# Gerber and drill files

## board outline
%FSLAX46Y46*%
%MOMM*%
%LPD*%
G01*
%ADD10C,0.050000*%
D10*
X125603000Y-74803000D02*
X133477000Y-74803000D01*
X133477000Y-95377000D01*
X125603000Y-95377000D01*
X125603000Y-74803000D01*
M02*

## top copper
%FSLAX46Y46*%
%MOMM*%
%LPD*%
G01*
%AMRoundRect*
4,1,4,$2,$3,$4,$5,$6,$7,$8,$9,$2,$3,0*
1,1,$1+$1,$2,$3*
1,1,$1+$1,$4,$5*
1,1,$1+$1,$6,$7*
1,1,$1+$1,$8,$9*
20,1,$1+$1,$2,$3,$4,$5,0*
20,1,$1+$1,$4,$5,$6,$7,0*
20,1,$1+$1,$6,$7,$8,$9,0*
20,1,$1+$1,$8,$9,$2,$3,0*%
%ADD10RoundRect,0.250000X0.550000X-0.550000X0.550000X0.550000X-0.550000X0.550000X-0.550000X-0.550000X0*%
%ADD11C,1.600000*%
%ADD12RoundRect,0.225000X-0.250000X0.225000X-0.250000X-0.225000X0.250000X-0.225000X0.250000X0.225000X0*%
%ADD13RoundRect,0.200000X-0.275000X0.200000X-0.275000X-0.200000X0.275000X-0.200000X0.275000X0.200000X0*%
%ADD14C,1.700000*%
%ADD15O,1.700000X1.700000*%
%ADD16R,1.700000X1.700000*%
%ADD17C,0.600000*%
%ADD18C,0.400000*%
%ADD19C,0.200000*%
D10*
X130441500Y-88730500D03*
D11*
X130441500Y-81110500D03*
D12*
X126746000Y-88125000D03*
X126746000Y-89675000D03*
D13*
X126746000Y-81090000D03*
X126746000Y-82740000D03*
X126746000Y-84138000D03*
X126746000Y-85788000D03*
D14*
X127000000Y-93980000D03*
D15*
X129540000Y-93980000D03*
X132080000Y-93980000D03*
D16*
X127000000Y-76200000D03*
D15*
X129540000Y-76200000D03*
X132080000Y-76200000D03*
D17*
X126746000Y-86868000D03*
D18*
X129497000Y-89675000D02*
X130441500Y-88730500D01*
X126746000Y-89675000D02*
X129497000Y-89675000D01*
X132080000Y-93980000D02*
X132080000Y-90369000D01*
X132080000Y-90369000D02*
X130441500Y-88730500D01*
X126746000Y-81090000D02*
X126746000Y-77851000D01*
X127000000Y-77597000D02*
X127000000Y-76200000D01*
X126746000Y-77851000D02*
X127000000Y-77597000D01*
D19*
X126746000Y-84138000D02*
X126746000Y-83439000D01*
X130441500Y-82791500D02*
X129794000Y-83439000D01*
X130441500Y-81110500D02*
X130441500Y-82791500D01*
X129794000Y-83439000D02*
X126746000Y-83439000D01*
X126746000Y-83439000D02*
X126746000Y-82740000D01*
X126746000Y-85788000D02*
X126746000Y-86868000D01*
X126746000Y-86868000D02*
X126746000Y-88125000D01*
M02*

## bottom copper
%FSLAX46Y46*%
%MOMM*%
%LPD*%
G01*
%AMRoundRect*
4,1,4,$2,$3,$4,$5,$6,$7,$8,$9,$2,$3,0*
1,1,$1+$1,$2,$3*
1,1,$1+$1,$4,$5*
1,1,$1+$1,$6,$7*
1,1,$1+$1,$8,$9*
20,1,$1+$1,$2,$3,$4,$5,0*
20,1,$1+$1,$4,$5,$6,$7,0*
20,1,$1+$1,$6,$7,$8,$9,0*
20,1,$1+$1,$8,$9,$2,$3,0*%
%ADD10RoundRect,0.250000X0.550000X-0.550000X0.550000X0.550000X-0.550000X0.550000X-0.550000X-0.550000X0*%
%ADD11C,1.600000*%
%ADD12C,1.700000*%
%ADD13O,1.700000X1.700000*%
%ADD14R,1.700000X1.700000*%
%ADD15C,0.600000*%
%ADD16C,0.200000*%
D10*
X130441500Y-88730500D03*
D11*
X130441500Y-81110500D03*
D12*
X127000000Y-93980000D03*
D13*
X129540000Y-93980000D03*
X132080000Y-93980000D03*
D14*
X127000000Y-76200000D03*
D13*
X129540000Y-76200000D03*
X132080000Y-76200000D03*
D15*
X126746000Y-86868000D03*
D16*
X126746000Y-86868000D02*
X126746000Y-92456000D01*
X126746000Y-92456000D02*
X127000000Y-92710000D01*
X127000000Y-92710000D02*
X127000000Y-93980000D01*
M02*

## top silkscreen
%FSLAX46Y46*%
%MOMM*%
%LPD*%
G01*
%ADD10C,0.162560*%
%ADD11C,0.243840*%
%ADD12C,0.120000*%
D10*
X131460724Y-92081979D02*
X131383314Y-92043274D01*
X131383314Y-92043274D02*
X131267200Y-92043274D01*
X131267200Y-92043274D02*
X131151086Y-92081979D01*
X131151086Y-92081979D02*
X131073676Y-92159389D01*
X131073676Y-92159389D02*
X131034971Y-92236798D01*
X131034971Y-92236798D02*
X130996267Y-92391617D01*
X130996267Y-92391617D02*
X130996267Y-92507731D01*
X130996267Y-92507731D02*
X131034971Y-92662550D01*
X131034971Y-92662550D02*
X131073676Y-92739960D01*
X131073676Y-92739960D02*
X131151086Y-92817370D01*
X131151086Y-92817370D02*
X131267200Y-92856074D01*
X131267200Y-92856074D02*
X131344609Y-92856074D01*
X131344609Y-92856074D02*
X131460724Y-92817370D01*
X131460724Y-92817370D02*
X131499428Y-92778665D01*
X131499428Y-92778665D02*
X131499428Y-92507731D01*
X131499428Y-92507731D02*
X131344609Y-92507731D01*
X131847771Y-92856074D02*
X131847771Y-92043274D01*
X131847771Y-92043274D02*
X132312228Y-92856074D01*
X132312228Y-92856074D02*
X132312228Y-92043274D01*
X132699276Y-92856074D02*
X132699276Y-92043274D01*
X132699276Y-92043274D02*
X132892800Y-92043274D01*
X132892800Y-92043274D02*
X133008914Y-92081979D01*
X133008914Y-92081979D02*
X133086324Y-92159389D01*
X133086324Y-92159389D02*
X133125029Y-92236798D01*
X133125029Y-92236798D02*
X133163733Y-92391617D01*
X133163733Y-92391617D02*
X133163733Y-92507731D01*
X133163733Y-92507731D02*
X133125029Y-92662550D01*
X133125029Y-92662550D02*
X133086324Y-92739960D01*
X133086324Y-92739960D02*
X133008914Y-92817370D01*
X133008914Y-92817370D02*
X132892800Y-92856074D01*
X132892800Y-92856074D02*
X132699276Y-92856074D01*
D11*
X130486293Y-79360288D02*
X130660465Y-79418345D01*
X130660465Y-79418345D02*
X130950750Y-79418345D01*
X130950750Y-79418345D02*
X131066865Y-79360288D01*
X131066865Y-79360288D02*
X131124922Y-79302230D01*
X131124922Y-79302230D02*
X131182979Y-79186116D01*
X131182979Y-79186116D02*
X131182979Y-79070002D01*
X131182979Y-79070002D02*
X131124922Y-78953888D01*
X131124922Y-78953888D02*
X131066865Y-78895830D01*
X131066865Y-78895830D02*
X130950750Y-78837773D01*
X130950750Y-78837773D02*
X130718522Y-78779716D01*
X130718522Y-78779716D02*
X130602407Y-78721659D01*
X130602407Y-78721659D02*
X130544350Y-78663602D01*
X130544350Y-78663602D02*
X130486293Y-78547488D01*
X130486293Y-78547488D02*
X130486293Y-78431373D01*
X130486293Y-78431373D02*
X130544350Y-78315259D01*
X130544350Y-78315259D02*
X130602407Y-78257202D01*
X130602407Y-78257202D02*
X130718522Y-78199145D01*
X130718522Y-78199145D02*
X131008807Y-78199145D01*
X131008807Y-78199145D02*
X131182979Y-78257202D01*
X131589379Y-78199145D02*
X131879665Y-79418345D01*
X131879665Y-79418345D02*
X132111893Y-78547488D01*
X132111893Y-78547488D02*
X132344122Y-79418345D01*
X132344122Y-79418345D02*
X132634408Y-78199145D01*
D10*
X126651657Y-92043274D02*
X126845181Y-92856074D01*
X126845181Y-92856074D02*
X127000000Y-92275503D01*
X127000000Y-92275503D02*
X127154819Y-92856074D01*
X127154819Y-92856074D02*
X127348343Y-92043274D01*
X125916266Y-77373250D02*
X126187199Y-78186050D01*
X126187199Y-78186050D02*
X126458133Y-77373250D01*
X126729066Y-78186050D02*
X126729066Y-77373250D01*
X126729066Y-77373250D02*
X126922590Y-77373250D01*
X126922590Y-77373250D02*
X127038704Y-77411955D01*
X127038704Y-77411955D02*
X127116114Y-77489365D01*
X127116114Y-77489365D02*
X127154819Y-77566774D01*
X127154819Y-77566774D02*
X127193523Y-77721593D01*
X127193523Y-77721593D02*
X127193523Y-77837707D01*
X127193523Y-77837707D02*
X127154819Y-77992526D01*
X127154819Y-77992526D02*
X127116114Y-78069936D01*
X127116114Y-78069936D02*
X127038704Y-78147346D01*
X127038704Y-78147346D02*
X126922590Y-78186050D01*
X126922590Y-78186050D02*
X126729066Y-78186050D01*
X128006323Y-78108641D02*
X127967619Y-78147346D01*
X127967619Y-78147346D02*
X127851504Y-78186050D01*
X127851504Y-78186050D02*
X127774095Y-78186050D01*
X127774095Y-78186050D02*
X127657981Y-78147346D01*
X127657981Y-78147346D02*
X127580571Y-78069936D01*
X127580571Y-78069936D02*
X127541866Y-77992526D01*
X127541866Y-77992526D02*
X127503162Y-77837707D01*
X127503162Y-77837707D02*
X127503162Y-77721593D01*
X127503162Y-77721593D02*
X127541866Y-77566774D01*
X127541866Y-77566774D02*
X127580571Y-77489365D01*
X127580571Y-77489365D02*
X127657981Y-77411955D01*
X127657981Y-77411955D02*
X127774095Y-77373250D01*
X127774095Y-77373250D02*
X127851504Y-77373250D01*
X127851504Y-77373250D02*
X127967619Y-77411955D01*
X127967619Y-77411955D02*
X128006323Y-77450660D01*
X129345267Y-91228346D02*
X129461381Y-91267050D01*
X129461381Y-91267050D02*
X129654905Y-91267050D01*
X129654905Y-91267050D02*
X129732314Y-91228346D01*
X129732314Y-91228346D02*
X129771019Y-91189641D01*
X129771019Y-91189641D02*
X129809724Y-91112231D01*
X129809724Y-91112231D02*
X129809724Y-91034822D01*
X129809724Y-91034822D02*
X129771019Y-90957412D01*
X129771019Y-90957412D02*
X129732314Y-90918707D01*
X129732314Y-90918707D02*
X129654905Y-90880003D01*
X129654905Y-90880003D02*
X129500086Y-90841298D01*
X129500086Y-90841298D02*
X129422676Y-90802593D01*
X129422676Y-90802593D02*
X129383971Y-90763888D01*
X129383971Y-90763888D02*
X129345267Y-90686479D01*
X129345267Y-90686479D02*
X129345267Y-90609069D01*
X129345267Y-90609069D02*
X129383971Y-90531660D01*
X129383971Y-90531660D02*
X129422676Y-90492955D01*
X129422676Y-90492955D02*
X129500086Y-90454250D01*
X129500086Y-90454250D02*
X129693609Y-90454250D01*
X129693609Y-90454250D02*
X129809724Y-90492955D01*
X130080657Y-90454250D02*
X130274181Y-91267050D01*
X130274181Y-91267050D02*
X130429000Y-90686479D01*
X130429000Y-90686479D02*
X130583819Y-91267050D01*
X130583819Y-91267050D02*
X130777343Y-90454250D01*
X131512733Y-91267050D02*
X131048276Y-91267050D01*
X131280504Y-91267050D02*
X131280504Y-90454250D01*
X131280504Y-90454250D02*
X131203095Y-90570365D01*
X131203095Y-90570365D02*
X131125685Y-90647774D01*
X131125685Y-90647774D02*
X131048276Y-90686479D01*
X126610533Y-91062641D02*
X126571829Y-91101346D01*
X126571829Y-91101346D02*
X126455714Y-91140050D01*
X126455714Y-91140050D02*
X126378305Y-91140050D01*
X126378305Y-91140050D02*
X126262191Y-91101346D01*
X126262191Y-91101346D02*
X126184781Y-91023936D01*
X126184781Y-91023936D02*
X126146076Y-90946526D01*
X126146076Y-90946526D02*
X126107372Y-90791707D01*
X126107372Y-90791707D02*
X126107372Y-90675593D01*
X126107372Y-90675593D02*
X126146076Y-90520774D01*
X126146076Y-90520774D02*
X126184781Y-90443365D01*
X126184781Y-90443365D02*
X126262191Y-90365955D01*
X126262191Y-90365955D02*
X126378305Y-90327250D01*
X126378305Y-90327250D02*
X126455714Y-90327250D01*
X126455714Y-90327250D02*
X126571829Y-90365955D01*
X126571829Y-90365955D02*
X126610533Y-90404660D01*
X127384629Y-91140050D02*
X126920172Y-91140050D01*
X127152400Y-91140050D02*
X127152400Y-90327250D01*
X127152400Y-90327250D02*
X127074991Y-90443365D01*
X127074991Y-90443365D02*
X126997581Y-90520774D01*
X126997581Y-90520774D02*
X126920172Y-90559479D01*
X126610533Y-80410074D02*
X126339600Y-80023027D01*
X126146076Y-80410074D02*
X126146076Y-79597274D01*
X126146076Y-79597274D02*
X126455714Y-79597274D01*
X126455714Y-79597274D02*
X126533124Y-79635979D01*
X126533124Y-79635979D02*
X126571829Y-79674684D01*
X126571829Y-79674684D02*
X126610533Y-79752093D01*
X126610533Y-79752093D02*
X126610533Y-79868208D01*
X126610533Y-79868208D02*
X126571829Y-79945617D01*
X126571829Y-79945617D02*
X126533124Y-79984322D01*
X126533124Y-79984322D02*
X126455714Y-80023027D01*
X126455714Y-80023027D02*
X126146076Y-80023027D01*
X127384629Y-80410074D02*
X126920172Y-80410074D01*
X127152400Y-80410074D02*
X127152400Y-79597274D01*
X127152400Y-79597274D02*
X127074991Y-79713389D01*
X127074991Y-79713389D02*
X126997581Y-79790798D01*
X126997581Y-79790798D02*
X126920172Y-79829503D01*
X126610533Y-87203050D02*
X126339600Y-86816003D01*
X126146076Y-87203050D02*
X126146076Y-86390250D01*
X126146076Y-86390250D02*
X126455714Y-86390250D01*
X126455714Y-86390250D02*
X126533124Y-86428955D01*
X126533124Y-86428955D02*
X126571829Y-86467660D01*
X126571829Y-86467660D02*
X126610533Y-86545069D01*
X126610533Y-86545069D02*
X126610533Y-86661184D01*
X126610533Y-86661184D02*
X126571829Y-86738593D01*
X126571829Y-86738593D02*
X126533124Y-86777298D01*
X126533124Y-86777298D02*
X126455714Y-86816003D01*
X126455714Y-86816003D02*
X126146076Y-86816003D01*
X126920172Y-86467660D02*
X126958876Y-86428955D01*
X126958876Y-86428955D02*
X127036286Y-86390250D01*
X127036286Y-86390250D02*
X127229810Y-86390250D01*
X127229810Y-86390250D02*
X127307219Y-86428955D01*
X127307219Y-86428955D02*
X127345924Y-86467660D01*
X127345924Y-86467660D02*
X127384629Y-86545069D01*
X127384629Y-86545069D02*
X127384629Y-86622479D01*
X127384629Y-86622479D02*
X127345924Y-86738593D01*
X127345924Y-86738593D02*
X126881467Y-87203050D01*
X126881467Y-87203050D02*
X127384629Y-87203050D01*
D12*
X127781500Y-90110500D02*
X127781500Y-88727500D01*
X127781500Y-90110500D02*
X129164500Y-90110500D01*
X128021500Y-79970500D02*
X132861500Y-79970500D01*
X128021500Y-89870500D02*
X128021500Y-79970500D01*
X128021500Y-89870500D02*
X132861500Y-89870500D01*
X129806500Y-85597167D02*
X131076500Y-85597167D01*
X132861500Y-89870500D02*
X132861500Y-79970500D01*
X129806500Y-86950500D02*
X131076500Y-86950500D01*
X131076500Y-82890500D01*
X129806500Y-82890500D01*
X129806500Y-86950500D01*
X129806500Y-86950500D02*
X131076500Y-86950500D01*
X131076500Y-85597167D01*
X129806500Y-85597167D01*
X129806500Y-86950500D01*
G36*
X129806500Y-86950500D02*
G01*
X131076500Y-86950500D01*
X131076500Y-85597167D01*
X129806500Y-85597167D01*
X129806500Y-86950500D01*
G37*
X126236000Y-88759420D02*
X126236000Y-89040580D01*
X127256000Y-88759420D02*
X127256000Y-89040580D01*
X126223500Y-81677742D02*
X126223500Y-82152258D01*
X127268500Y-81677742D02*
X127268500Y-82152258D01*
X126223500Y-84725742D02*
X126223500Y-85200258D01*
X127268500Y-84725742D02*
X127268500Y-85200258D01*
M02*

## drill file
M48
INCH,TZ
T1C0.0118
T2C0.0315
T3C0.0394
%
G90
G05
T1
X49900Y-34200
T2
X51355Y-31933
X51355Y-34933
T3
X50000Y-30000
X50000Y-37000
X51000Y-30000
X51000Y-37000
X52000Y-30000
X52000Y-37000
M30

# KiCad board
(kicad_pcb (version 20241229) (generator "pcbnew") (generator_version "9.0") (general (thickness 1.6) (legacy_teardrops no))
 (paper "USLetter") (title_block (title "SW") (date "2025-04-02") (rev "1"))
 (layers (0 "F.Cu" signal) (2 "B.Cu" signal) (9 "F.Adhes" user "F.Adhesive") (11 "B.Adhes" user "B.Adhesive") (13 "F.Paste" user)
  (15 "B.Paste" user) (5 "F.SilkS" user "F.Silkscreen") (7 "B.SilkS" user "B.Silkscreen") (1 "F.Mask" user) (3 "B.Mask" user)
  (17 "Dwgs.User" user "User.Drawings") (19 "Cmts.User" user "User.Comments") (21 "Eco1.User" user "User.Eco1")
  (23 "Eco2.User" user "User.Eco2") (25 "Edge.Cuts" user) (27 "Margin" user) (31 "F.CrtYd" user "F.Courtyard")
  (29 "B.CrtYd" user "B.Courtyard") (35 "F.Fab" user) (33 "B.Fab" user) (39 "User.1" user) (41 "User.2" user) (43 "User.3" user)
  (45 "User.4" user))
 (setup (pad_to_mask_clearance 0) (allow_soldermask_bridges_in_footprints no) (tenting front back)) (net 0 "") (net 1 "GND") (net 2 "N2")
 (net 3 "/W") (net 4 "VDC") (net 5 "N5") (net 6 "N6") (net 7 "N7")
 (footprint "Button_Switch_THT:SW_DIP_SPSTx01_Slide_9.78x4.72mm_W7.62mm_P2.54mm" (layer "F.Cu") (at 130.4415 88.7305 90)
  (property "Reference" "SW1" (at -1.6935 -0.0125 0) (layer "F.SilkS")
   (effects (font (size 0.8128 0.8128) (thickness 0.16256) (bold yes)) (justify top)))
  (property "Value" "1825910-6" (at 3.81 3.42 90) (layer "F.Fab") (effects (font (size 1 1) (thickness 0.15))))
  (fp_line (start -1.38 -2.66) (end 0.003 -2.66) (stroke (width 0.12) (type solid)) (layer "F.SilkS"))
  (fp_line (start -1.38 -2.66) (end -1.38 -1.277) (stroke (width 0.12) (type solid)) (layer "F.SilkS"))
  (fp_line (start 8.76 -2.42) (end 8.76 2.42) (stroke (width 0.12) (type solid)) (layer "F.SilkS"))
  (fp_line (start -1.14 -2.42) (end 8.76 -2.42) (stroke (width 0.12) (type solid)) (layer "F.SilkS"))
  (fp_line (start -1.14 -2.42) (end -1.14 2.42) (stroke (width 0.12) (type solid)) (layer "F.SilkS"))
  (fp_line (start 3.133333 -0.635) (end 3.133333 0.635) (stroke (width 0.12) (type solid)) (layer "F.SilkS"))
  (fp_line (start -1.14 2.42) (end 8.76 2.42) (stroke (width 0.12) (type solid)) (layer "F.SilkS"))
  (fp_rect (start 1.78 -0.635) (end 5.84 0.635) (stroke (width 0.12) (type solid)) (fill no) (layer "F.SilkS"))
  (fp_rect (start 1.78 -0.635) (end 3.133333 0.635) (stroke (width 0.12) (type solid)) (fill yes) (layer "F.SilkS"))
  (pad "1" thru_hole roundrect (at 0 0 90) (size 1.6 1.6) (drill 0.8) (layers "*.Cu" "*.Mask") (remove_unused_layers no)
   (roundrect_rratio 0.15625) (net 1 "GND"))
  (pad "2" thru_hole circle (at 7.62 0 90) (size 1.6 1.6) (drill 0.8) (layers "*.Cu" "*.Mask") (remove_unused_layers no) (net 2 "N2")))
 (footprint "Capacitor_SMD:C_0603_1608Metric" (layer "F.Cu") (at 126.746 88.9 -90)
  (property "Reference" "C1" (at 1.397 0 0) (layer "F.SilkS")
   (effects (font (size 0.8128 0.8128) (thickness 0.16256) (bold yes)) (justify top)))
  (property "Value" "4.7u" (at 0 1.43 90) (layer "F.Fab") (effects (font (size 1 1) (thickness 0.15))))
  (fp_line (start -0.14058 0.51) (end 0.14058 0.51) (stroke (width 0.12) (type solid)) (layer "F.SilkS"))
  (fp_line (start -0.14058 -0.51) (end 0.14058 -0.51) (stroke (width 0.12) (type solid)) (layer "F.SilkS"))
  (pad "1" smd roundrect (at -0.775 0 270) (size 0.9 0.95) (layers "F.Cu" "F.Mask" "F.Paste") (roundrect_rratio 0.25) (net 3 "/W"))
  (pad "2" smd roundrect (at 0.775 0 270) (size 0.9 0.95) (layers "F.Cu" "F.Mask" "F.Paste") (roundrect_rratio 0.25) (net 1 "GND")))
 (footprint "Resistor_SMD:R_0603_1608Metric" (layer "F.Cu") (at 126.746 81.915 -90)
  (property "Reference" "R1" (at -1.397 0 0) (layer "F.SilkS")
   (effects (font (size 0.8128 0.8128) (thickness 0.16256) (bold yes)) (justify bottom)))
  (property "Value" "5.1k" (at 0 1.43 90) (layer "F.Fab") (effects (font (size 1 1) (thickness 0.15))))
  (fp_line (start -0.237258 0.5225) (end 0.237258 0.5225) (stroke (width 0.12) (type solid)) (layer "F.SilkS"))
  (fp_line (start -0.237258 -0.5225) (end 0.237258 -0.5225) (stroke (width 0.12) (type solid)) (layer "F.SilkS"))
  (pad "1" smd roundrect (at -0.825 0 270) (size 0.8 0.95) (layers "F.Cu" "F.Mask" "F.Paste") (roundrect_rratio 0.25) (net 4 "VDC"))
  (pad "2" smd roundrect (at 0.825 0 270) (size 0.8 0.95) (layers "F.Cu" "F.Mask" "F.Paste") (roundrect_rratio 0.25) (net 2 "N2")))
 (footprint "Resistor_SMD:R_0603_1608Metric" (layer "F.Cu") (at 126.746 84.963 -90)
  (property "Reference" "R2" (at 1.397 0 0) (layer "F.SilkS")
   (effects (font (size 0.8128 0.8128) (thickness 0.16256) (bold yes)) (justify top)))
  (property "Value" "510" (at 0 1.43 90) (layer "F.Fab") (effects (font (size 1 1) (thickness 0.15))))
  (fp_line (start -0.237258 0.5225) (end 0.237258 0.5225) (stroke (width 0.12) (type solid)) (layer "F.SilkS"))
  (fp_line (start -0.237258 -0.5225) (end 0.237258 -0.5225) (stroke (width 0.12) (type solid)) (layer "F.SilkS"))
  (pad "1" smd roundrect (at -0.825 0 270) (size 0.8 0.95) (layers "F.Cu" "F.Mask" "F.Paste") (roundrect_rratio 0.25) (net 2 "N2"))
  (pad "2" smd roundrect (at 0.825 0 270) (size 0.8 0.95) (layers "F.Cu" "F.Mask" "F.Paste") (roundrect_rratio 0.25) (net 3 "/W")))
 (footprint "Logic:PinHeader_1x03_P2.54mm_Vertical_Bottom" (layer "B.Cu") (at 127 93.98 -90)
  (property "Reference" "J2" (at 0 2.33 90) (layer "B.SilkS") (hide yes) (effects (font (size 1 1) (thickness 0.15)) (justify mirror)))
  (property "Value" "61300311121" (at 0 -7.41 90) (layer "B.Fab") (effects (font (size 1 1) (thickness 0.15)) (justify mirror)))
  (pad "1" thru_hole circle (at 0 0 270) (size 1.7 1.7) (drill 1) (layers "*.Cu" "*.Mask") (remove_unused_layers no) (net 3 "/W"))
  (pad "2" thru_hole oval (at 0 -2.54 270) (size 1.7 1.7) (drill 1) (layers "*.Cu" "*.Mask") (remove_unused_layers no) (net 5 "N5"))
  (pad "3" thru_hole oval (at 0 -5.08 270) (size 1.7 1.7) (drill 1) (layers "*.Cu" "*.Mask") (remove_unused_layers no) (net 1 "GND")))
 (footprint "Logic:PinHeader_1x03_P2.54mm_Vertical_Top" (layer "B.Cu") (at 127 76.2 -90)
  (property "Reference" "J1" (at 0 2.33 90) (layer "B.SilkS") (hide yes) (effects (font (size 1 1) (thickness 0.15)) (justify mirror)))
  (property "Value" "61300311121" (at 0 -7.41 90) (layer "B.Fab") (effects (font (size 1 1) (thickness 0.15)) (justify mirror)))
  (pad "1" thru_hole rect (at 0 0 270) (size 1.7 1.7) (drill 1) (layers "*.Cu" "*.Mask") (remove_unused_layers no) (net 4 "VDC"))
  (pad "2" thru_hole oval (at 0 -2.54 270) (size 1.7 1.7) (drill 1) (layers "*.Cu" "*.Mask") (remove_unused_layers no) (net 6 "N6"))
  (pad "3" thru_hole oval (at 0 -5.08 270) (size 1.7 1.7) (drill 1) (layers "*.Cu" "*.Mask") (remove_unused_layers no) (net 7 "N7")))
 (gr_rect (start 125.603 74.803) (end 133.477 95.377) (stroke (width 0.05) (type default)) (fill no) (layer "Edge.Cuts"))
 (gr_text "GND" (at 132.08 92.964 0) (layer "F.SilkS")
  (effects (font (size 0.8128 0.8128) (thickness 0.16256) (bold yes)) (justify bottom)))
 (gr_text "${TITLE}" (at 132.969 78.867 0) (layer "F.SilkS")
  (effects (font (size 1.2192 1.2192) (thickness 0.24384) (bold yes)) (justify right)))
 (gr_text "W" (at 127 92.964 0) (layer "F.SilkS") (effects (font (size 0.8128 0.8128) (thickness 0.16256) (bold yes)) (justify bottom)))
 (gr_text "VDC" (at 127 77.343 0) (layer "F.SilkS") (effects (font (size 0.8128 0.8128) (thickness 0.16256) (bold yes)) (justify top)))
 (segment (start 129.497 89.675) (end 130.4415 88.7305) (width 0.4) (layer "F.Cu") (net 1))
 (segment (start 126.746 89.675) (end 129.497 89.675) (width 0.4) (layer "F.Cu") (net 1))
 (segment (start 132.08 93.98) (end 132.08 90.369) (width 0.4) (layer "F.Cu") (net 1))
 (segment (start 132.08 90.369) (end 130.4415 88.7305) (width 0.4) (layer "F.Cu") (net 1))
 (segment (start 126.746 81.09) (end 126.746 77.851) (width 0.4) (layer "F.Cu") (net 4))
 (segment (start 127 77.597) (end 127 76.2) (width 0.4) (layer "F.Cu") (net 4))
 (segment (start 126.746 77.851) (end 127 77.597) (width 0.4) (layer "F.Cu") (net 4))
 (segment (start 126.746 84.138) (end 126.746 83.439) (width 0.2) (layer "F.Cu") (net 2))
 (segment (start 130.4415 82.7915) (end 129.794 83.439) (width 0.2) (layer "F.Cu") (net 2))
 (segment (start 130.4415 81.1105) (end 130.4415 82.7915) (width 0.2) (layer "F.Cu") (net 2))
 (segment (start 129.794 83.439) (end 126.746 83.439) (width 0.2) (layer "F.Cu") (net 2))
 (segment (start 126.746 83.439) (end 126.746 82.74) (width 0.2) (layer "F.Cu") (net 2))
 (segment (start 126.746 85.788) (end 126.746 86.868) (width 0.2) (layer "F.Cu") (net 3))
 (segment (start 126.746 86.868) (end 126.746 88.125) (width 0.2) (layer "F.Cu") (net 3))
 (via (at 126.746 86.868) (size 0.6) (drill 0.3) (layers "F.Cu" "B.Cu") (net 3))
 (segment (start 126.746 86.868) (end 126.746 92.456) (width 0.2) (layer "B.Cu") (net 3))
 (segment (start 126.746 92.456) (end 127 92.71) (width 0.2) (layer "B.Cu") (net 3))
 (segment (start 127 92.71) (end 127 93.98) (width 0.2) (layer "B.Cu") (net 3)))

